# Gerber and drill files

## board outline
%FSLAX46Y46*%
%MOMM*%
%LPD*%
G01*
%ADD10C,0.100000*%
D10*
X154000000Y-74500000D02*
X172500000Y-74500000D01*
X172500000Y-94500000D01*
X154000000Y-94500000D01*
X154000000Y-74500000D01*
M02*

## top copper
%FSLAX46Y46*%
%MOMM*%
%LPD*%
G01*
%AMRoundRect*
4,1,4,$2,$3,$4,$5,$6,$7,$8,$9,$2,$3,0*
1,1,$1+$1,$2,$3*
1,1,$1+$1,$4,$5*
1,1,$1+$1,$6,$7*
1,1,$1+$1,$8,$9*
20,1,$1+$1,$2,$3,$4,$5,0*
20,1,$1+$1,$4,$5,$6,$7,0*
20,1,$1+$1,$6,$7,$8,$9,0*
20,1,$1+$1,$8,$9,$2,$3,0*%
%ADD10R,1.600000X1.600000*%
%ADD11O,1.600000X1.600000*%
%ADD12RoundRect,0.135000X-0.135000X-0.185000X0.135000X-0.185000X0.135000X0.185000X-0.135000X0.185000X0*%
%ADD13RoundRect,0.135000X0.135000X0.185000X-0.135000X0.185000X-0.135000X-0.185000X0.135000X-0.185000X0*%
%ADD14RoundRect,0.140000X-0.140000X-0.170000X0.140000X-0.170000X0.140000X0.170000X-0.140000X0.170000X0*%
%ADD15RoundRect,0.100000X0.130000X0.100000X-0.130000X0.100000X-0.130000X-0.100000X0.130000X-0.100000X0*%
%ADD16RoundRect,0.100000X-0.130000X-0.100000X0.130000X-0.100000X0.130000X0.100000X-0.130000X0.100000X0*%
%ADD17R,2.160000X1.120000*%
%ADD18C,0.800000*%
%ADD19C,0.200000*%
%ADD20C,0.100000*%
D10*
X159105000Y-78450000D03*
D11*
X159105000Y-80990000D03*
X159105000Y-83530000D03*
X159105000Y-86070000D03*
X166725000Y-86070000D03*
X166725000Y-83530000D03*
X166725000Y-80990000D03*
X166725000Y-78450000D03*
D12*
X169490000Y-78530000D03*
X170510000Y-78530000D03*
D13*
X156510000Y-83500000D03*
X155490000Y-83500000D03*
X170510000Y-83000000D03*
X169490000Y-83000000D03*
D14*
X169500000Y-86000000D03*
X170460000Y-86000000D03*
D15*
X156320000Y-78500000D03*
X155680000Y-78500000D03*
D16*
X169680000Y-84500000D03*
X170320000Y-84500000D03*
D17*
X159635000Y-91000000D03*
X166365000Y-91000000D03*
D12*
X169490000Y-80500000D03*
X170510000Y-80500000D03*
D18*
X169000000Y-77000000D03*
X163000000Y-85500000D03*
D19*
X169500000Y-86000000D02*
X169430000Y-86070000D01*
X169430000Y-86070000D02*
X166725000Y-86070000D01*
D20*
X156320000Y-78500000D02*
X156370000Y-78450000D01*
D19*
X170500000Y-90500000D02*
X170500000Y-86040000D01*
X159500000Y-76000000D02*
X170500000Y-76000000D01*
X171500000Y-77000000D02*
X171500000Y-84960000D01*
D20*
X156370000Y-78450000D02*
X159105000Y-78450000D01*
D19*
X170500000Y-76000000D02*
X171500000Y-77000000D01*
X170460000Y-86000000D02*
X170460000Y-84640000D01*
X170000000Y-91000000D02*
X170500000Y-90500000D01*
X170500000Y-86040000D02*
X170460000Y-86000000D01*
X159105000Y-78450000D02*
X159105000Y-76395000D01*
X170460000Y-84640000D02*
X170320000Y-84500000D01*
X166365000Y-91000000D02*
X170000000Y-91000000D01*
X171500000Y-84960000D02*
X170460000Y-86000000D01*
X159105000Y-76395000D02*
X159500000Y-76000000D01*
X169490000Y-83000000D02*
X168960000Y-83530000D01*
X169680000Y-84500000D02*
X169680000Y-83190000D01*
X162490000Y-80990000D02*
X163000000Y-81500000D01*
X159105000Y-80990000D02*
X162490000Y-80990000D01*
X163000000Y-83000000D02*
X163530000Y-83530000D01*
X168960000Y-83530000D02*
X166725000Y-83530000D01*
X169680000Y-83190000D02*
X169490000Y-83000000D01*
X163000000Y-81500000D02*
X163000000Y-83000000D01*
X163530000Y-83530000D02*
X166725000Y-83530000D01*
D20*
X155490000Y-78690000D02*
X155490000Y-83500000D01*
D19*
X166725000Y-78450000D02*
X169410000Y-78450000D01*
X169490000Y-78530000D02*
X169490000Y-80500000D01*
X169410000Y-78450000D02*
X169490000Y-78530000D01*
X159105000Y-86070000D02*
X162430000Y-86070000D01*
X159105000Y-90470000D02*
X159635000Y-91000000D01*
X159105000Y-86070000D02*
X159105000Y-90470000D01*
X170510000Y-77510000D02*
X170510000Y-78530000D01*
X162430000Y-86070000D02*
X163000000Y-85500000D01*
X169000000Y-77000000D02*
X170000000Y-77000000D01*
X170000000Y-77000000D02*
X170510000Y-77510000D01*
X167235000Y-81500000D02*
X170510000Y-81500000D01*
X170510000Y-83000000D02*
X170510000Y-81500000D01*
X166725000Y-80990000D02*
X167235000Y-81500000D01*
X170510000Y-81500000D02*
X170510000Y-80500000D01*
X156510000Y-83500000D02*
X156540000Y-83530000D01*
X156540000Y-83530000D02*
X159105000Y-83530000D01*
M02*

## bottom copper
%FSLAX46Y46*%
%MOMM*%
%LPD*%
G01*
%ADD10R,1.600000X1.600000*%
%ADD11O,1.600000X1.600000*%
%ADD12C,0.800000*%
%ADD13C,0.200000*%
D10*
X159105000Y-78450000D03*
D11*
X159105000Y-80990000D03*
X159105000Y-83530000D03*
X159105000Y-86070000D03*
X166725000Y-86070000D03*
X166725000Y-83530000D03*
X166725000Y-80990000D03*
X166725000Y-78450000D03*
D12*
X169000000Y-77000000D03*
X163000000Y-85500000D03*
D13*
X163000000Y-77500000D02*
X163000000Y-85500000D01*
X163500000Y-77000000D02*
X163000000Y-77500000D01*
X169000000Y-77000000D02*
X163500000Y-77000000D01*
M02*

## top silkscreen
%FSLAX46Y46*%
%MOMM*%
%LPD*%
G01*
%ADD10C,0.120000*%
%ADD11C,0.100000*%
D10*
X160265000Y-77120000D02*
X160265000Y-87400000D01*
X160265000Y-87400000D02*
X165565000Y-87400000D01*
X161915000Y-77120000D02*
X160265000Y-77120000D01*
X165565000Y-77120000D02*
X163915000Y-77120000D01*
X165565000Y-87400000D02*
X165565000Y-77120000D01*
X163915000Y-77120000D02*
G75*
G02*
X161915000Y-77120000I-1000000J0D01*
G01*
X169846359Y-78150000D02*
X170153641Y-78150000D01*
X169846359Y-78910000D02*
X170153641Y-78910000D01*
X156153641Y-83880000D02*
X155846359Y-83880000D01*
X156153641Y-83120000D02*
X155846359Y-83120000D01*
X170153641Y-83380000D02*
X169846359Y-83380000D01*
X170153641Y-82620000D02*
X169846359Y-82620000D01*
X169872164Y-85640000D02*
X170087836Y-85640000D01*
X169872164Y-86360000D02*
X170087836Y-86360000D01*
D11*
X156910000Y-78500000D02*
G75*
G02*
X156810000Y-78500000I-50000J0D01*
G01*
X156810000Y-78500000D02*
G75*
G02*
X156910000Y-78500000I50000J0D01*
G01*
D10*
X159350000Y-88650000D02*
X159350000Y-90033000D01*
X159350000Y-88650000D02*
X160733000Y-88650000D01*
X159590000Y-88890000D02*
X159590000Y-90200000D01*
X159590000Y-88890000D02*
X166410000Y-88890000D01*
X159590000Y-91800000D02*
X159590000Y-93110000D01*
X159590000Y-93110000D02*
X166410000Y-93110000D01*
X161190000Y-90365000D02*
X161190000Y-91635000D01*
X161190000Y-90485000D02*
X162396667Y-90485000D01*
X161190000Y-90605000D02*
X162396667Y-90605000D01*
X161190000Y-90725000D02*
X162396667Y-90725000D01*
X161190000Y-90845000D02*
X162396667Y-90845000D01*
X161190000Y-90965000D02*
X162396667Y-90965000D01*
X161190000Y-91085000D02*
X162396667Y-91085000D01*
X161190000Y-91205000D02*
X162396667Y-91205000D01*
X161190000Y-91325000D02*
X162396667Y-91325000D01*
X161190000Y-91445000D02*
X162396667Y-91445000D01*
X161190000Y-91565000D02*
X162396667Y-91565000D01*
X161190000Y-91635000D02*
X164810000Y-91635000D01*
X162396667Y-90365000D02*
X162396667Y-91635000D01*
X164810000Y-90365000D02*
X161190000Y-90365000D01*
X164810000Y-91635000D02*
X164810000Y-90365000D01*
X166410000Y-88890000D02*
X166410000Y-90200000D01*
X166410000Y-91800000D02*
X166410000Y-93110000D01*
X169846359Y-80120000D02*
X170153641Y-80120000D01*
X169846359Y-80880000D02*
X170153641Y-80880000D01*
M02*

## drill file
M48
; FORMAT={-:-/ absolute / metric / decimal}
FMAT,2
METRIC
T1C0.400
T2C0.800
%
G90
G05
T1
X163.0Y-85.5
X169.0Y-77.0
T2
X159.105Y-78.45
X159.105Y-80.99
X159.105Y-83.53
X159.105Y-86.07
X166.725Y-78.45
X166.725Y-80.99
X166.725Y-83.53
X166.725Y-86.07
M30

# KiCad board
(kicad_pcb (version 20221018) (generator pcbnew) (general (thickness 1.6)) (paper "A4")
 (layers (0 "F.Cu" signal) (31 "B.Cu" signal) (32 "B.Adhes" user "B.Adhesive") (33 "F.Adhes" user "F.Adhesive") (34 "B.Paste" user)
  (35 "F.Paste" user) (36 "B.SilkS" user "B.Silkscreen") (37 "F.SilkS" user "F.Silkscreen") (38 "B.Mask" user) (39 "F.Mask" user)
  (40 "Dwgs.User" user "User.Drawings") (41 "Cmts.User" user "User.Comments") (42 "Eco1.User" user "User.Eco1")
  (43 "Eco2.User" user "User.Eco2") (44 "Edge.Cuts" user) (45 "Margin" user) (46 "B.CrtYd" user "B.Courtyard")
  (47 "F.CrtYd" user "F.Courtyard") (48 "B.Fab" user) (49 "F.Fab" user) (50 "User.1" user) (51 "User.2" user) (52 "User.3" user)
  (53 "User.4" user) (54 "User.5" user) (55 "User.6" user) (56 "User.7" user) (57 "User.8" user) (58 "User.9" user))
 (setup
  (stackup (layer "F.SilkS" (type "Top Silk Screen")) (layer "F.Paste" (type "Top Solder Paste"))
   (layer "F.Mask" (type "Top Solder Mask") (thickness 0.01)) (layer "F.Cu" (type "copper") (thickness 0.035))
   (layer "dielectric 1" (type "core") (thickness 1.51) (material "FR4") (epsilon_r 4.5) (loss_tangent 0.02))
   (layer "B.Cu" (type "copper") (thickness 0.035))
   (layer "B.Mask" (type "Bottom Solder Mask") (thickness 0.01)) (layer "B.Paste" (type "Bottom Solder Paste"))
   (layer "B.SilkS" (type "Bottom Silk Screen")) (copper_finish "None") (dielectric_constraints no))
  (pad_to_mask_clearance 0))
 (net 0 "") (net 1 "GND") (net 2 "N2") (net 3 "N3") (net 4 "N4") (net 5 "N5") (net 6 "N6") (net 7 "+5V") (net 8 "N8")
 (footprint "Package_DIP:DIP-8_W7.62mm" (layer "F.Cu") (at 159.105 78.45)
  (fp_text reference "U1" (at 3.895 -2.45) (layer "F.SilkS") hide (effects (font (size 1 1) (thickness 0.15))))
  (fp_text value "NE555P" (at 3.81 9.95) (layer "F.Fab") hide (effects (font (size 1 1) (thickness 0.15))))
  (fp_line (start 1.16 -1.33) (end 1.16 8.95) (stroke (width 0.12) (type solid)) (layer "F.SilkS"))
  (fp_line (start 1.16 8.95) (end 6.46 8.95) (stroke (width 0.12) (type solid)) (layer "F.SilkS"))
  (fp_line (start 2.81 -1.33) (end 1.16 -1.33) (stroke (width 0.12) (type solid)) (layer "F.SilkS"))
  (fp_line (start 6.46 -1.33) (end 4.81 -1.33) (stroke (width 0.12) (type solid)) (layer "F.SilkS"))
  (fp_line (start 6.46 8.95) (end 6.46 -1.33) (stroke (width 0.12) (type solid)) (layer "F.SilkS"))
  (fp_arc (start 4.81 -1.33) (mid 3.81 -0.33) (end 2.81 -1.33) (stroke (width 0.12) (type solid)) (layer "F.SilkS"))
  (pad "1" thru_hole rect (at 0 0) (size 1.6 1.6) (drill 0.8) (layers "*.Cu" "*.Mask") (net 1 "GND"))
  (pad "2" thru_hole oval (at 0 2.54) (size 1.6 1.6) (drill 0.8) (layers "*.Cu" "*.Mask") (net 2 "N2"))
  (pad "3" thru_hole oval (at 0 5.08) (size 1.6 1.6) (drill 0.8) (layers "*.Cu" "*.Mask") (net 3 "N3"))
  (pad "4" thru_hole oval (at 0 7.62) (size 1.6 1.6) (drill 0.8) (layers "*.Cu" "*.Mask") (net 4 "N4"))
  (pad "5" thru_hole oval (at 7.62 7.62) (size 1.6 1.6) (drill 0.8) (layers "*.Cu" "*.Mask") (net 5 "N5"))
  (pad "6" thru_hole oval (at 7.62 5.08) (size 1.6 1.6) (drill 0.8) (layers "*.Cu" "*.Mask") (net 2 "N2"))
  (pad "7" thru_hole oval (at 7.62 2.54) (size 1.6 1.6) (drill 0.8) (layers "*.Cu" "*.Mask") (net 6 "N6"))
  (pad "8" thru_hole oval (at 7.62 0) (size 1.6 1.6) (drill 0.8) (layers "*.Cu" "*.Mask") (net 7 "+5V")))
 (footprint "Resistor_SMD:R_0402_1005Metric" (layer "F.Cu") (at 170 78.53)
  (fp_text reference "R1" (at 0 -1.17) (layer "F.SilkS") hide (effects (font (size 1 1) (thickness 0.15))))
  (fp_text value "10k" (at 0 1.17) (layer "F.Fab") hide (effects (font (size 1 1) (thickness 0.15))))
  (fp_line (start -0.153641 -0.38) (end 0.153641 -0.38) (stroke (width 0.12) (type solid)) (layer "F.SilkS"))
  (fp_line (start -0.153641 0.38) (end 0.153641 0.38) (stroke (width 0.12) (type solid)) (layer "F.SilkS"))
  (pad "1" smd roundrect (at -0.51 0) (size 0.54 0.64) (layers "F.Cu" "F.Paste" "F.Mask") (roundrect_rratio 0.25) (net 7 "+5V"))
  (pad "2" smd roundrect (at 0.51 0) (size 0.54 0.64) (layers "F.Cu" "F.Paste" "F.Mask") (roundrect_rratio 0.25) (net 4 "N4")))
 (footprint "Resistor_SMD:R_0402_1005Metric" (layer "F.Cu") (at 156 83.5 180)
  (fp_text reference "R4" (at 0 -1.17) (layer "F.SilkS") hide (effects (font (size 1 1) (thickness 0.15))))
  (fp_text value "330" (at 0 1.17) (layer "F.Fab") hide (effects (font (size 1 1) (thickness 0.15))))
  (fp_line (start -0.153641 -0.38) (end 0.153641 -0.38) (stroke (width 0.12) (type solid)) (layer "F.SilkS"))
  (fp_line (start -0.153641 0.38) (end 0.153641 0.38) (stroke (width 0.12) (type solid)) (layer "F.SilkS"))
  (pad "1" smd roundrect (at -0.51 0 180) (size 0.54 0.64) (layers "F.Cu" "F.Paste" "F.Mask") (roundrect_rratio 0.25) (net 3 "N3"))
  (pad "2" smd roundrect (at 0.51 0 180) (size 0.54 0.64) (layers "F.Cu" "F.Paste" "F.Mask") (roundrect_rratio 0.25) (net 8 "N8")))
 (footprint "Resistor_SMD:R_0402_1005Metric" (layer "F.Cu") (at 170 83 180)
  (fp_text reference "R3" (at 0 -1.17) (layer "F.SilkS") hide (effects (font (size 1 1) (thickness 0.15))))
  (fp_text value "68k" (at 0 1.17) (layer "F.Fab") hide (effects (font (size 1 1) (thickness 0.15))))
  (fp_line (start -0.153641 -0.38) (end 0.153641 -0.38) (stroke (width 0.12) (type solid)) (layer "F.SilkS"))
  (fp_line (start -0.153641 0.38) (end 0.153641 0.38) (stroke (width 0.12) (type solid)) (layer "F.SilkS"))
  (pad "1" smd roundrect (at -0.51 0 180) (size 0.54 0.64) (layers "F.Cu" "F.Paste" "F.Mask") (roundrect_rratio 0.25) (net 6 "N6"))
  (pad "2" smd roundrect (at 0.51 0 180) (size 0.54 0.64) (layers "F.Cu" "F.Paste" "F.Mask") (roundrect_rratio 0.25) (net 2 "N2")))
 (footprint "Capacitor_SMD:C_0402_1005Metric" (layer "F.Cu") (at 169.98 86)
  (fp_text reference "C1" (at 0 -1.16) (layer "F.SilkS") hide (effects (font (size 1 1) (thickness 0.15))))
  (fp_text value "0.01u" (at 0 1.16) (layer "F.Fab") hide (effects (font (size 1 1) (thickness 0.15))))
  (fp_line (start -0.107836 -0.36) (end 0.107836 -0.36) (stroke (width 0.12) (type solid)) (layer "F.SilkS"))
  (fp_line (start -0.107836 0.36) (end 0.107836 0.36) (stroke (width 0.12) (type solid)) (layer "F.SilkS"))
  (pad "1" smd roundrect (at -0.48 0) (size 0.56 0.62) (layers "F.Cu" "F.Paste" "F.Mask") (roundrect_rratio 0.25) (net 5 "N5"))
  (pad "2" smd roundrect (at 0.48 0) (size 0.56 0.62) (layers "F.Cu" "F.Paste" "F.Mask") (roundrect_rratio 0.25) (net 1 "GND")))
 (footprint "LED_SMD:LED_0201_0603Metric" (layer "F.Cu") (at 156 78.5 180)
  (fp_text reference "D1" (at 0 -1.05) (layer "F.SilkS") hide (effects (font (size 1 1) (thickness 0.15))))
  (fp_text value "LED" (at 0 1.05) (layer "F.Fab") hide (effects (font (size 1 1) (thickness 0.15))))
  (fp_circle (center -0.86 0) (end -0.81 0) (stroke (width 0.1) (type solid)) (fill none) (layer "F.SilkS"))
  (pad "" smd roundrect (at -0.345 0 180) (size 0.318 0.36) (layers "F.Paste") (roundrect_rratio 0.25))
  (pad "" smd roundrect (at 0.345 0 180) (size 0.318 0.36) (layers "F.Paste") (roundrect_rratio 0.25))
  (pad "1" smd roundrect (at -0.32 0 180) (size 0.46 0.4) (layers "F.Cu" "F.Mask") (roundrect_rratio 0.25) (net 1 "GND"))
  (pad "2" smd roundrect (at 0.32 0 180) (size 0.46 0.4) (layers "F.Cu" "F.Mask") (roundrect_rratio 0.25) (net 8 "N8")))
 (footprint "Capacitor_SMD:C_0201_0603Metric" (layer "F.Cu") (at 170 84.5)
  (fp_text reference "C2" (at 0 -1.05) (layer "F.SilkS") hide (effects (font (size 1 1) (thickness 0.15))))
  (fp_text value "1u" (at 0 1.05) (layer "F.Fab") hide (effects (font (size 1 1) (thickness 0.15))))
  (pad "" smd roundrect (at -0.345 0) (size 0.318 0.36) (layers "F.Paste") (roundrect_rratio 0.25))
  (pad "" smd roundrect (at 0.345 0) (size 0.318 0.36) (layers "F.Paste") (roundrect_rratio 0.25))
  (pad "1" smd roundrect (at -0.32 0) (size 0.46 0.4) (layers "F.Cu" "F.Mask") (roundrect_rratio 0.25) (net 2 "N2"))
  (pad "2" smd roundrect (at 0.32 0) (size 0.46 0.4) (layers "F.Cu" "F.Mask") (roundrect_rratio 0.25) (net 1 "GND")))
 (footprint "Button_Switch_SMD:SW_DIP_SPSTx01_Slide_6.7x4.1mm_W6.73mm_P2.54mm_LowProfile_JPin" (layer "F.Cu") (at 163 91)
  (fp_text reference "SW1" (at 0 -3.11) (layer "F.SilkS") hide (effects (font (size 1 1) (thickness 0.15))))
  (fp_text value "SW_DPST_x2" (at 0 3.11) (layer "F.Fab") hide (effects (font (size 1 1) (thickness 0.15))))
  (fp_line (start -3.65 -2.35) (end -3.65 -0.967) (stroke (width 0.12) (type solid)) (layer "F.SilkS"))
  (fp_line (start -3.65 -2.35) (end -2.267 -2.35) (stroke (width 0.12) (type solid)) (layer "F.SilkS"))
  (fp_line (start -3.41 -2.11) (end -3.41 -0.8) (stroke (width 0.12) (type solid)) (layer "F.SilkS"))
  (fp_line (start -3.41 -2.11) (end 3.41 -2.11) (stroke (width 0.12) (type solid)) (layer "F.SilkS"))
  (fp_line (start -3.41 0.8) (end -3.41 2.11) (stroke (width 0.12) (type solid)) (layer "F.SilkS"))
  (fp_line (start -3.41 2.11) (end 3.41 2.11) (stroke (width 0.12) (type solid)) (layer "F.SilkS"))
  (fp_line (start -1.81 -0.635) (end -1.81 0.635) (stroke (width 0.12) (type solid)) (layer "F.SilkS"))
  (fp_line (start -1.81 -0.515) (end -0.603333 -0.515) (stroke (width 0.12) (type solid)) (layer "F.SilkS"))
  (fp_line (start -1.81 -0.395) (end -0.603333 -0.395) (stroke (width 0.12) (type solid)) (layer "F.SilkS"))
  (fp_line (start -1.81 -0.275) (end -0.603333 -0.275) (stroke (width 0.12) (type solid)) (layer "F.SilkS"))
  (fp_line (start -1.81 -0.155) (end -0.603333 -0.155) (stroke (width 0.12) (type solid)) (layer "F.SilkS"))
  (fp_line (start -1.81 -0.035) (end -0.603333 -0.035) (stroke (width 0.12) (type solid)) (layer "F.SilkS"))
  (fp_line (start -1.81 0.085) (end -0.603333 0.085) (stroke (width 0.12) (type solid)) (layer "F.SilkS"))
  (fp_line (start -1.81 0.205) (end -0.603333 0.205) (stroke (width 0.12) (type solid)) (layer "F.SilkS"))
  (fp_line (start -1.81 0.325) (end -0.603333 0.325) (stroke (width 0.12) (type solid)) (layer "F.SilkS"))
  (fp_line (start -1.81 0.445) (end -0.603333 0.445) (stroke (width 0.12) (type solid)) (layer "F.SilkS"))
  (fp_line (start -1.81 0.565) (end -0.603333 0.565) (stroke (width 0.12) (type solid)) (layer "F.SilkS"))
  (fp_line (start -1.81 0.635) (end 1.81 0.635) (stroke (width 0.12) (type solid)) (layer "F.SilkS"))
  (fp_line (start -0.603333 -0.635) (end -0.603333 0.635) (stroke (width 0.12) (type solid)) (layer "F.SilkS"))
  (fp_line (start 1.81 -0.635) (end -1.81 -0.635) (stroke (width 0.12) (type solid)) (layer "F.SilkS"))
  (fp_line (start 1.81 0.635) (end 1.81 -0.635) (stroke (width 0.12) (type solid)) (layer "F.SilkS"))
  (fp_line (start 3.41 -2.11) (end 3.41 -0.8) (stroke (width 0.12) (type solid)) (layer "F.SilkS"))
  (fp_line (start 3.41 0.8) (end 3.41 2.11) (stroke (width 0.12) (type solid)) (layer "F.SilkS"))
  (pad "1" smd rect (at -3.365 0) (size 2.16 1.12) (layers "F.Cu" "F.Paste" "F.Mask") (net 4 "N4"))
  (pad "2" smd rect (at 3.365 0) (size 2.16 1.12) (layers "F.Cu" "F.Paste" "F.Mask") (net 1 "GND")))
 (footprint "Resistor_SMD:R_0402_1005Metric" (layer "F.Cu") (at 170 80.5)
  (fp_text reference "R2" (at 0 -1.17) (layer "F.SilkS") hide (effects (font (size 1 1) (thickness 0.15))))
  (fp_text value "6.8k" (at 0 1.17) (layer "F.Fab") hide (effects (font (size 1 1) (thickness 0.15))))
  (fp_line (start -0.153641 -0.38) (end 0.153641 -0.38) (stroke (width 0.12) (type solid)) (layer "F.SilkS"))
  (fp_line (start -0.153641 0.38) (end 0.153641 0.38) (stroke (width 0.12) (type solid)) (layer "F.SilkS"))
  (pad "1" smd roundrect (at -0.51 0) (size 0.54 0.64) (layers "F.Cu" "F.Paste" "F.Mask") (roundrect_rratio 0.25) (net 7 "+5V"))
  (pad "2" smd roundrect (at 0.51 0) (size 0.54 0.64) (layers "F.Cu" "F.Paste" "F.Mask") (roundrect_rratio 0.25) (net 6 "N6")))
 (gr_rect (start 154 74.5) (end 172.5 94.5) (stroke (width 0.1) (type default)) (fill none) (layer "Edge.Cuts"))
 (segment (start 169.5 86) (end 169.43 86.07) (width 0.2) (layer "F.Cu") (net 5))
 (segment (start 169.43 86.07) (end 166.725 86.07) (width 0.2) (layer "F.Cu") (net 5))
 (segment (start 156.32 78.5) (end 156.37 78.45) (width 0.1) (layer "F.Cu") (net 1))
 (segment (start 170.5 90.5) (end 170.5 86.04) (width 0.2) (layer "F.Cu") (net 1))
 (segment (start 159.5 76) (end 170.5 76) (width 0.2) (layer "F.Cu") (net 1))
 (segment (start 171.5 77) (end 171.5 84.96) (width 0.2) (layer "F.Cu") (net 1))
 (segment (start 156.37 78.45) (end 159.105 78.45) (width 0.1) (layer "F.Cu") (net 1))
 (segment (start 170.5 76) (end 171.5 77) (width 0.2) (layer "F.Cu") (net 1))
 (segment (start 170.46 86) (end 170.46 84.64) (width 0.2) (layer "F.Cu") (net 1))
 (segment (start 170 91) (end 170.5 90.5) (width 0.2) (layer "F.Cu") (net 1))
 (segment (start 170.5 86.04) (end 170.46 86) (width 0.2) (layer "F.Cu") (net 1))
 (segment (start 159.105 78.45) (end 159.105 76.395) (width 0.2) (layer "F.Cu") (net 1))
 (segment (start 170.46 84.64) (end 170.32 84.5) (width 0.2) (layer "F.Cu") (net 1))
 (segment (start 166.365 91) (end 170 91) (width 0.2) (layer "F.Cu") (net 1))
 (segment (start 171.5 84.96) (end 170.46 86) (width 0.2) (layer "F.Cu") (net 1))
 (segment (start 159.105 76.395) (end 159.5 76) (width 0.2) (layer "F.Cu") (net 1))
 (segment (start 169.49 83) (end 168.96 83.53) (width 0.2) (layer "F.Cu") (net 2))
 (segment (start 169.68 84.5) (end 169.68 83.19) (width 0.2) (layer "F.Cu") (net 2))
 (segment (start 162.49 80.99) (end 163 81.5) (width 0.2) (layer "F.Cu") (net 2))
 (segment (start 159.105 80.99) (end 162.49 80.99) (width 0.2) (layer "F.Cu") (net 2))
 (segment (start 163 83) (end 163.53 83.53) (width 0.2) (layer "F.Cu") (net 2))
 (segment (start 168.96 83.53) (end 166.725 83.53) (width 0.2) (layer "F.Cu") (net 2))
 (segment (start 169.68 83.19) (end 169.49 83) (width 0.2) (layer "F.Cu") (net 2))
 (segment (start 163 81.5) (end 163 83) (width 0.2) (layer "F.Cu") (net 2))
 (segment (start 163.53 83.53) (end 166.725 83.53) (width 0.2) (layer "F.Cu") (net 2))
 (segment (start 155.49 78.69) (end 155.49 83.5) (width 0.1) (layer "F.Cu") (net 8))
 (segment (start 166.725 78.45) (end 169.41 78.45) (width 0.2) (layer "F.Cu") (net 7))
 (segment (start 169.49 78.53) (end 169.49 80.5) (width 0.2) (layer "F.Cu") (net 7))
 (segment (start 169.41 78.45) (end 169.49 78.53) (width 0.2) (layer "F.Cu") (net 7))
 (segment (start 159.105 86.07) (end 162.43 86.07) (width 0.2) (layer "F.Cu") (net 4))
 (segment (start 159.105 90.47) (end 159.635 91) (width 0.2) (layer "F.Cu") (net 4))
 (segment (start 159.105 86.07) (end 159.105 90.47) (width 0.2) (layer "F.Cu") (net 4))
 (segment (start 170.51 77.51) (end 170.51 78.53) (width 0.2) (layer "F.Cu") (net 4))
 (segment (start 162.43 86.07) (end 163 85.5) (width 0.2) (layer "F.Cu") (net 4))
 (segment (start 169 77) (end 170 77) (width 0.2) (layer "F.Cu") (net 4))
 (segment (start 170 77) (end 170.51 77.51) (width 0.2) (layer "F.Cu") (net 4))
 (via (at 169 77) (size 0.8) (drill 0.4) (layers "F.Cu" "B.Cu") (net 4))
 (via (at 163 85.5) (size 0.8) (drill 0.4) (layers "F.Cu" "B.Cu") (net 4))
 (segment (start 163 77.5) (end 163 85.5) (width 0.2) (layer "B.Cu") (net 4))
 (segment (start 163.5 77) (end 163 77.5) (width 0.2) (layer "B.Cu") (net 4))
 (segment (start 169 77) (end 163.5 77) (width 0.2) (layer "B.Cu") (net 4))
 (segment (start 167.235 81.5) (end 170.51 81.5) (width 0.2) (layer "F.Cu") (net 6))
 (segment (start 170.51 83) (end 170.51 81.5) (width 0.2) (layer "F.Cu") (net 6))
 (segment (start 166.725 80.99) (end 167.235 81.5) (width 0.2) (layer "F.Cu") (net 6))
 (segment (start 170.51 81.5) (end 170.51 80.5) (width 0.2) (layer "F.Cu") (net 6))
 (segment (start 156.51 83.5) (end 156.54 83.53) (width 0.2) (layer "F.Cu") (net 3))
 (segment (start 156.54 83.53) (end 159.105 83.53) (width 0.2) (layer "F.Cu") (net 3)))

